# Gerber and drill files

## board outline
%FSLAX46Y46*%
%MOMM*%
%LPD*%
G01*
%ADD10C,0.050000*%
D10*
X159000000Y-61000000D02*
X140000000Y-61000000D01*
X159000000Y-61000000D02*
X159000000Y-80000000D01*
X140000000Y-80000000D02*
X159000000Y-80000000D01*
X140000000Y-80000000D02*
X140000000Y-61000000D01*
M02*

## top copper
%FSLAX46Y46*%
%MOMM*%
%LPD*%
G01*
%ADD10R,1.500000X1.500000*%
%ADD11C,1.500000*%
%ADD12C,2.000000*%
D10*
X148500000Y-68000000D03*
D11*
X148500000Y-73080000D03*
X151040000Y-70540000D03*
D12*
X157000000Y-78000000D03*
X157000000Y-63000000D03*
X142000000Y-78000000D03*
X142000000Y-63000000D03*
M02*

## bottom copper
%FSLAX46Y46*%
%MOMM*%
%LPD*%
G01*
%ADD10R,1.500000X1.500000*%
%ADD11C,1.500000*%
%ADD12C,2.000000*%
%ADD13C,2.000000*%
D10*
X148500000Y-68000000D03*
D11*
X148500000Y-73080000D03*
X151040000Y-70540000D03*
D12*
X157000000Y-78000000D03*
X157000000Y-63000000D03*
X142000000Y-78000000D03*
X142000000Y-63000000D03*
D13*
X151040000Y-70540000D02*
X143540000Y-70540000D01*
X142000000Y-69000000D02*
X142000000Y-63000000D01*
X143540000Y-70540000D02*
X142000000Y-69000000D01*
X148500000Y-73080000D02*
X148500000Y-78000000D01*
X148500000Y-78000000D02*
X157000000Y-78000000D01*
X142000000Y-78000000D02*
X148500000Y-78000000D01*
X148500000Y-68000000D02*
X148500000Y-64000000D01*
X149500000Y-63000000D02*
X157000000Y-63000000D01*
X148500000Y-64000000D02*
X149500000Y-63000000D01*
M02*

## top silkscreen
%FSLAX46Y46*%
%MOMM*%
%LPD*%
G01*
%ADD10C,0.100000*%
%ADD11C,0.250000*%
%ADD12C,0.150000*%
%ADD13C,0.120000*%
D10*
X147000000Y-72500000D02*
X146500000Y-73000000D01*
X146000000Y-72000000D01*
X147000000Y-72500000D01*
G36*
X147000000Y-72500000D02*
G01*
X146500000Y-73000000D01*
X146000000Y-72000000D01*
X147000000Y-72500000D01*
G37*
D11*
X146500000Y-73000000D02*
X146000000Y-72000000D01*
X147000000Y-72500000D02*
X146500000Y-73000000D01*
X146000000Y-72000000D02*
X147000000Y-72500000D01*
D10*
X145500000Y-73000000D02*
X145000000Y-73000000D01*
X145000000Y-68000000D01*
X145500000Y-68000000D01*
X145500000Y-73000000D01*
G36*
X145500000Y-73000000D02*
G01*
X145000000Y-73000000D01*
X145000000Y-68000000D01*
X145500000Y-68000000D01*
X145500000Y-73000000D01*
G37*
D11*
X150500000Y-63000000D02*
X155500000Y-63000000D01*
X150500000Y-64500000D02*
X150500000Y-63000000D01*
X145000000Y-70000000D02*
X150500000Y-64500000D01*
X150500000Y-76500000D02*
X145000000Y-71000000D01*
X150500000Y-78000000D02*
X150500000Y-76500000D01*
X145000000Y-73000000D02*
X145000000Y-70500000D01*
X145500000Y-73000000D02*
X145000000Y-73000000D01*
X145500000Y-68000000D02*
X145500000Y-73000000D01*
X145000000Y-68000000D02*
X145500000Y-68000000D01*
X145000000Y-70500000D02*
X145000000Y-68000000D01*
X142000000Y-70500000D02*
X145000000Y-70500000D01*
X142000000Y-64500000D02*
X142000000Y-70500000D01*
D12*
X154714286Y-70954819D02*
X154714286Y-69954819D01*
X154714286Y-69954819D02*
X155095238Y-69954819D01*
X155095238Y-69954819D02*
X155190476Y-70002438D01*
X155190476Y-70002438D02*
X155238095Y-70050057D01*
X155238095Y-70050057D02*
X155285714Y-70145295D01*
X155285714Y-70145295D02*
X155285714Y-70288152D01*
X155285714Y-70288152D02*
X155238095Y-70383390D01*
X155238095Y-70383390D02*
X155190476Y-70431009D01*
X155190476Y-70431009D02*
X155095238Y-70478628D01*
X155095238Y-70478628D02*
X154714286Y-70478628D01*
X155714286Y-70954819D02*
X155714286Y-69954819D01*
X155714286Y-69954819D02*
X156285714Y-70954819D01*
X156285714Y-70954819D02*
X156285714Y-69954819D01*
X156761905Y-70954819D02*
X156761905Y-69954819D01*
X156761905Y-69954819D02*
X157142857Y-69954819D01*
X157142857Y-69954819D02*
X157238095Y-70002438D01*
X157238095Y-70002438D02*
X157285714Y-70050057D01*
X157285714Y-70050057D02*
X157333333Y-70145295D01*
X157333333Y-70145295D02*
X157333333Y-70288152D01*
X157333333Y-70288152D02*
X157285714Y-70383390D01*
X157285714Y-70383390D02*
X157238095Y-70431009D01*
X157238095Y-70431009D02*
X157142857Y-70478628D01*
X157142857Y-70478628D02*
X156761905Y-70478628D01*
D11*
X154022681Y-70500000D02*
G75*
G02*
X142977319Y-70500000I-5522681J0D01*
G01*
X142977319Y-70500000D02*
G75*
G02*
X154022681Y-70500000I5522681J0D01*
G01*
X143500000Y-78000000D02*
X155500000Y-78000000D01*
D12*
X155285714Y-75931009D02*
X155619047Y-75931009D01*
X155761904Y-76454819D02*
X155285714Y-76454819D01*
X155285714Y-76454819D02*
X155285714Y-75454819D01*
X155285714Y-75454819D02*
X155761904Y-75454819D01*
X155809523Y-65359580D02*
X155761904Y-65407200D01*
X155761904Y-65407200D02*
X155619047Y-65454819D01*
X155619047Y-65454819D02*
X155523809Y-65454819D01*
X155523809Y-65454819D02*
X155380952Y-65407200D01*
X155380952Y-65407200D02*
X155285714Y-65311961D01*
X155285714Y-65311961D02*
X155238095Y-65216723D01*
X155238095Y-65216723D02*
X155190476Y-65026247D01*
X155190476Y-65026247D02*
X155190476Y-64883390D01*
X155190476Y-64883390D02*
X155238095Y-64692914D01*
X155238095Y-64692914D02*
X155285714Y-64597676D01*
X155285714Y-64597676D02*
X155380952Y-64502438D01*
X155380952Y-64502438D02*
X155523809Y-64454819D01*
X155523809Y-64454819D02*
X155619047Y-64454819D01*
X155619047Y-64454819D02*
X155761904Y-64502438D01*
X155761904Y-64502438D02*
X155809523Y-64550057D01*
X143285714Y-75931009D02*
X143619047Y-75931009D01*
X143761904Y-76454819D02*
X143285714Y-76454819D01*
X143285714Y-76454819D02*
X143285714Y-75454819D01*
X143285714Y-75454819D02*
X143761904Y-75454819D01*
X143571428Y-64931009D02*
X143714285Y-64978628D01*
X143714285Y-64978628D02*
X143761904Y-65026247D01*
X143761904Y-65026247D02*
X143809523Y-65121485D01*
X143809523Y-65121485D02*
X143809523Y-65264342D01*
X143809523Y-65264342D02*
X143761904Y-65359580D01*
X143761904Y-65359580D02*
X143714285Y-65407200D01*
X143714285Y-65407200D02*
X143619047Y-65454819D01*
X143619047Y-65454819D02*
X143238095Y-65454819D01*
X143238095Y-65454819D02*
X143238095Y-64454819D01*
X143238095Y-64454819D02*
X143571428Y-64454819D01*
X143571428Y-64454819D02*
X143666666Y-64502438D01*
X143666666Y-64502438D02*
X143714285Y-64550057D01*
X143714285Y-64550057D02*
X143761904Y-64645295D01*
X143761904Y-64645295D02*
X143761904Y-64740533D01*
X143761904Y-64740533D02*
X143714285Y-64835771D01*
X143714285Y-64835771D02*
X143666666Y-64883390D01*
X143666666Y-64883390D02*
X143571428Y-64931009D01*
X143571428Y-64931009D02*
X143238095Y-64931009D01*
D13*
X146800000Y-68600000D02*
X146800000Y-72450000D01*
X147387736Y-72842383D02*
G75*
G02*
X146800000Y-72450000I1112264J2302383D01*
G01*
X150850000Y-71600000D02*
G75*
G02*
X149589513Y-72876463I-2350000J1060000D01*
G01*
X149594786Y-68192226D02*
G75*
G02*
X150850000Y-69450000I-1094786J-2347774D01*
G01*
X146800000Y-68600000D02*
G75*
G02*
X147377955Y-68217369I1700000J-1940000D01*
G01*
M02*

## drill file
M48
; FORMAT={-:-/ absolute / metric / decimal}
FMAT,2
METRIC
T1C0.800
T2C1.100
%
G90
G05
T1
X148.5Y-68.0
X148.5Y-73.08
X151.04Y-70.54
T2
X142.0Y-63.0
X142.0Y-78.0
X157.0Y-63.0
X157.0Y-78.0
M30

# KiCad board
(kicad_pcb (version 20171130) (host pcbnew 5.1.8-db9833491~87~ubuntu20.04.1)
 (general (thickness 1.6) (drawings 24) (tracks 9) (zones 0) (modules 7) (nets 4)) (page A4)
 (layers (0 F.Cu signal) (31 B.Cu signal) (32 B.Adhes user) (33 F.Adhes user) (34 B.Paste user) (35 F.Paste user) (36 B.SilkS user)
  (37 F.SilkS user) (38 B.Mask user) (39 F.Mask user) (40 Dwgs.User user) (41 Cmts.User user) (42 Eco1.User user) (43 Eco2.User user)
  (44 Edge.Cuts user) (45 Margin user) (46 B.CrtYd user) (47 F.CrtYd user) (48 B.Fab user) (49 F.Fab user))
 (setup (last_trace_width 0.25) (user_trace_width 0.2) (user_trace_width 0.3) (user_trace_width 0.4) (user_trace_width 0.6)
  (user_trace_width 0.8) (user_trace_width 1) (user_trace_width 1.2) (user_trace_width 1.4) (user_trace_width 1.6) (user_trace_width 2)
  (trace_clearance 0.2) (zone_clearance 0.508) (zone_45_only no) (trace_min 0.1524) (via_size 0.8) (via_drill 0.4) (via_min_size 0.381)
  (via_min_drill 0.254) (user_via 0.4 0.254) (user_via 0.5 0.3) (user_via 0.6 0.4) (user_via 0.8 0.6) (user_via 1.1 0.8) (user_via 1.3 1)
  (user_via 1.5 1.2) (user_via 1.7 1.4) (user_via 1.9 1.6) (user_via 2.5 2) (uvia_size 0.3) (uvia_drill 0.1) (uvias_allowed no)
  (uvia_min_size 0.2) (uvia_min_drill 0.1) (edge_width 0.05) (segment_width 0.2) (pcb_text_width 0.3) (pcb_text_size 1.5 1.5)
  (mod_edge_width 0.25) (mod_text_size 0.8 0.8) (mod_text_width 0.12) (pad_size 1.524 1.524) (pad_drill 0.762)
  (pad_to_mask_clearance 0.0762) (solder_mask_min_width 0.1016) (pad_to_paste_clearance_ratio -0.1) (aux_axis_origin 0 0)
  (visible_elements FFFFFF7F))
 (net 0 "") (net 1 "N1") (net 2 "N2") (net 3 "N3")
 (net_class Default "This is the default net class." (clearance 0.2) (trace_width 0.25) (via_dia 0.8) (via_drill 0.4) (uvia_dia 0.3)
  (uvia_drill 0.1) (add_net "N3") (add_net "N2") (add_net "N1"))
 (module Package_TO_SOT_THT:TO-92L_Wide (layer F.Cu) (at 148.5 68 270)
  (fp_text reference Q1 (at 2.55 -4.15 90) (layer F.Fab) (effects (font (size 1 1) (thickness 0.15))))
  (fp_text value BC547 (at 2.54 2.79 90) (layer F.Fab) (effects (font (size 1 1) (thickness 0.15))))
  (fp_line (start 0.6 1.7) (end 4.45 1.7) (layer F.SilkS) (width 0.12))
  (fp_arc (start 2.54 0) (end 4.45 1.7) (angle -15.88591585) (layer F.SilkS) (width 0.12))
  (fp_arc (start 2.54 0) (end 3.6 -2.35) (angle 40.72153779) (layer F.SilkS) (width 0.12))
  (fp_arc (start 2.54 0) (end 1.45 -2.35) (angle -40.11670855) (layer F.SilkS) (width 0.12))
  (fp_arc (start 2.54 0) (end 0.6 1.7) (angle 15.44288892) (layer F.SilkS) (width 0.12))
  (pad 1 thru_hole rect (at 0 0 270) (size 1.5 1.5) (drill 0.8) (layers *.Cu *.Mask) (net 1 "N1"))
  (pad 3 thru_hole circle (at 5.08 0 270) (size 1.5 1.5) (drill 0.8) (layers *.Cu *.Mask) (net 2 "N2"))
  (pad 2 thru_hole circle (at 2.54 -2.54 270) (size 1.5 1.5) (drill 0.8) (layers *.Cu *.Mask) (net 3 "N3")))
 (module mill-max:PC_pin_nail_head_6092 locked (layer F.Cu) (at 157 78)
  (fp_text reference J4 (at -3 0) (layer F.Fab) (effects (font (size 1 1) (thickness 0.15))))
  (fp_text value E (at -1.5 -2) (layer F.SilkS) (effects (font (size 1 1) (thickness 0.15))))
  (pad 1 thru_hole circle (at 0 0) (size 2 2) (drill 1.1) (layers *.Cu *.Mask) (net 2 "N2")))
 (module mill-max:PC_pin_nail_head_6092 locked (layer F.Cu) (at 157 63)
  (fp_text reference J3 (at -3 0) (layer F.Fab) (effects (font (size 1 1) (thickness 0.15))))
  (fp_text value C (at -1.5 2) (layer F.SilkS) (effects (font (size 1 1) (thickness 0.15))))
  (pad 1 thru_hole circle (at 0 0) (size 2 2) (drill 1.1) (layers *.Cu *.Mask) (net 1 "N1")))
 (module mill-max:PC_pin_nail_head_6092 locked (layer F.Cu) (at 142 78)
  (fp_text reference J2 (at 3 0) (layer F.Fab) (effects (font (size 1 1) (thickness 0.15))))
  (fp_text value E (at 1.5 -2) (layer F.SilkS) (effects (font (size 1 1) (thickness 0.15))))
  (pad 1 thru_hole circle (at 0 0) (size 2 2) (drill 1.1) (layers *.Cu *.Mask) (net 2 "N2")))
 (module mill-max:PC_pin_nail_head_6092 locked (layer F.Cu) (at 142 63)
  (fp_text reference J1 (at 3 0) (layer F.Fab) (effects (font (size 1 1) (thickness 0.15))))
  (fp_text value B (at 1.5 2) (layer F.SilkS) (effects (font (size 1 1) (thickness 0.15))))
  (pad 1 thru_hole circle (at 0 0) (size 2 2) (drill 1.1) (layers *.Cu *.Mask) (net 3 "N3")))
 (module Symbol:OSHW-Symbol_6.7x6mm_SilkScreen (layer B.Cu) (at 155.5 70.5 270)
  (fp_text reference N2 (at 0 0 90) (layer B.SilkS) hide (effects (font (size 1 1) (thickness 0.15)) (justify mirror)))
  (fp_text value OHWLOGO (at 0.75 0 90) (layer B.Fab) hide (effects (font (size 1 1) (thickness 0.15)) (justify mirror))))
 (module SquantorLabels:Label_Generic (layer B.Cu) (at 141.5 71.5 90)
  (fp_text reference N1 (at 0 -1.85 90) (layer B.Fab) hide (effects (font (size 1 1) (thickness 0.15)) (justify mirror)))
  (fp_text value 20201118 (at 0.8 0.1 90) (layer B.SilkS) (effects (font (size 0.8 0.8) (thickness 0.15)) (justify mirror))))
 (gr_poly (pts (xy 147 72.5) (xy 146.5 73) (xy 146 72)) (layer F.SilkS) (width 0.1))
 (gr_line (start 146.5 73) (end 146 72) (layer F.SilkS) (width 0.25))
 (gr_line (start 147 72.5) (end 146.5 73) (layer F.SilkS) (width 0.25))
 (gr_line (start 146 72) (end 147 72.5) (layer F.SilkS) (width 0.25))
 (gr_poly (pts (xy 145.5 73) (xy 145 73) (xy 145 68) (xy 145.5 68)) (layer F.SilkS) (width 0.1))
 (gr_line (start 150.5 63) (end 155.5 63) (layer F.SilkS) (width 0.25))
 (gr_line (start 150.5 64.5) (end 150.5 63) (layer F.SilkS) (width 0.25))
 (gr_line (start 145 70) (end 150.5 64.5) (layer F.SilkS) (width 0.25))
 (gr_line (start 150.5 76.5) (end 145 71) (layer F.SilkS) (width 0.25))
 (gr_line (start 150.5 78) (end 150.5 76.5) (layer F.SilkS) (width 0.25))
 (gr_line (start 145 73) (end 145 70.5) (layer F.SilkS) (width 0.25))
 (gr_line (start 145.5 73) (end 145 73) (layer F.SilkS) (width 0.25))
 (gr_line (start 145.5 68) (end 145.5 73) (layer F.SilkS) (width 0.25))
 (gr_line (start 145 68) (end 145.5 68) (layer F.SilkS) (width 0.25))
 (gr_line (start 145 70.5) (end 145 68) (layer F.SilkS) (width 0.25))
 (gr_line (start 142 70.5) (end 145 70.5) (layer F.SilkS) (width 0.25))
 (gr_line (start 142 64.5) (end 142 70.5) (layer F.SilkS) (width 0.25))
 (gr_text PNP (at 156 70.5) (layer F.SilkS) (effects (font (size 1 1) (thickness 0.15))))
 (gr_circle (center 148.5 70.5) (end 154 71) (layer F.SilkS) (width 0.25))
 (gr_line (start 143.5 78) (end 155.5 78) (layer F.SilkS) (width 0.25))
 (gr_line (start 159 61) (end 140 61) (layer Edge.Cuts) (width 0.05))
 (gr_line (start 159 61) (end 159 80) (layer Edge.Cuts) (width 0.05))
 (gr_line (start 140 80) (end 159 80) (layer Edge.Cuts) (width 0.05))
 (gr_line (start 140 80) (end 140 61) (layer Edge.Cuts) (width 0.05))
 (segment (start 151.04 70.54) (end 143.54 70.54) (width 2) (layer B.Cu) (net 3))
 (segment (start 142 69) (end 142 63) (width 2) (layer B.Cu) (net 3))
 (segment (start 143.54 70.54) (end 142 69) (width 2) (layer B.Cu) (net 3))
 (segment (start 148.5 73.08) (end 148.5 78) (width 2) (layer B.Cu) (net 2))
 (segment (start 148.5 78) (end 157 78) (width 2) (layer B.Cu) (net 2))
 (segment (start 142 78) (end 148.5 78) (width 2) (layer B.Cu) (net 2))
 (segment (start 148.5 68) (end 148.5 64) (width 2) (layer B.Cu) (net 1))
 (segment (start 149.5 63) (end 157 63) (width 2) (layer B.Cu) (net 1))
 (segment (start 148.5 64) (end 149.5 63) (width 2) (layer B.Cu) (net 1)))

